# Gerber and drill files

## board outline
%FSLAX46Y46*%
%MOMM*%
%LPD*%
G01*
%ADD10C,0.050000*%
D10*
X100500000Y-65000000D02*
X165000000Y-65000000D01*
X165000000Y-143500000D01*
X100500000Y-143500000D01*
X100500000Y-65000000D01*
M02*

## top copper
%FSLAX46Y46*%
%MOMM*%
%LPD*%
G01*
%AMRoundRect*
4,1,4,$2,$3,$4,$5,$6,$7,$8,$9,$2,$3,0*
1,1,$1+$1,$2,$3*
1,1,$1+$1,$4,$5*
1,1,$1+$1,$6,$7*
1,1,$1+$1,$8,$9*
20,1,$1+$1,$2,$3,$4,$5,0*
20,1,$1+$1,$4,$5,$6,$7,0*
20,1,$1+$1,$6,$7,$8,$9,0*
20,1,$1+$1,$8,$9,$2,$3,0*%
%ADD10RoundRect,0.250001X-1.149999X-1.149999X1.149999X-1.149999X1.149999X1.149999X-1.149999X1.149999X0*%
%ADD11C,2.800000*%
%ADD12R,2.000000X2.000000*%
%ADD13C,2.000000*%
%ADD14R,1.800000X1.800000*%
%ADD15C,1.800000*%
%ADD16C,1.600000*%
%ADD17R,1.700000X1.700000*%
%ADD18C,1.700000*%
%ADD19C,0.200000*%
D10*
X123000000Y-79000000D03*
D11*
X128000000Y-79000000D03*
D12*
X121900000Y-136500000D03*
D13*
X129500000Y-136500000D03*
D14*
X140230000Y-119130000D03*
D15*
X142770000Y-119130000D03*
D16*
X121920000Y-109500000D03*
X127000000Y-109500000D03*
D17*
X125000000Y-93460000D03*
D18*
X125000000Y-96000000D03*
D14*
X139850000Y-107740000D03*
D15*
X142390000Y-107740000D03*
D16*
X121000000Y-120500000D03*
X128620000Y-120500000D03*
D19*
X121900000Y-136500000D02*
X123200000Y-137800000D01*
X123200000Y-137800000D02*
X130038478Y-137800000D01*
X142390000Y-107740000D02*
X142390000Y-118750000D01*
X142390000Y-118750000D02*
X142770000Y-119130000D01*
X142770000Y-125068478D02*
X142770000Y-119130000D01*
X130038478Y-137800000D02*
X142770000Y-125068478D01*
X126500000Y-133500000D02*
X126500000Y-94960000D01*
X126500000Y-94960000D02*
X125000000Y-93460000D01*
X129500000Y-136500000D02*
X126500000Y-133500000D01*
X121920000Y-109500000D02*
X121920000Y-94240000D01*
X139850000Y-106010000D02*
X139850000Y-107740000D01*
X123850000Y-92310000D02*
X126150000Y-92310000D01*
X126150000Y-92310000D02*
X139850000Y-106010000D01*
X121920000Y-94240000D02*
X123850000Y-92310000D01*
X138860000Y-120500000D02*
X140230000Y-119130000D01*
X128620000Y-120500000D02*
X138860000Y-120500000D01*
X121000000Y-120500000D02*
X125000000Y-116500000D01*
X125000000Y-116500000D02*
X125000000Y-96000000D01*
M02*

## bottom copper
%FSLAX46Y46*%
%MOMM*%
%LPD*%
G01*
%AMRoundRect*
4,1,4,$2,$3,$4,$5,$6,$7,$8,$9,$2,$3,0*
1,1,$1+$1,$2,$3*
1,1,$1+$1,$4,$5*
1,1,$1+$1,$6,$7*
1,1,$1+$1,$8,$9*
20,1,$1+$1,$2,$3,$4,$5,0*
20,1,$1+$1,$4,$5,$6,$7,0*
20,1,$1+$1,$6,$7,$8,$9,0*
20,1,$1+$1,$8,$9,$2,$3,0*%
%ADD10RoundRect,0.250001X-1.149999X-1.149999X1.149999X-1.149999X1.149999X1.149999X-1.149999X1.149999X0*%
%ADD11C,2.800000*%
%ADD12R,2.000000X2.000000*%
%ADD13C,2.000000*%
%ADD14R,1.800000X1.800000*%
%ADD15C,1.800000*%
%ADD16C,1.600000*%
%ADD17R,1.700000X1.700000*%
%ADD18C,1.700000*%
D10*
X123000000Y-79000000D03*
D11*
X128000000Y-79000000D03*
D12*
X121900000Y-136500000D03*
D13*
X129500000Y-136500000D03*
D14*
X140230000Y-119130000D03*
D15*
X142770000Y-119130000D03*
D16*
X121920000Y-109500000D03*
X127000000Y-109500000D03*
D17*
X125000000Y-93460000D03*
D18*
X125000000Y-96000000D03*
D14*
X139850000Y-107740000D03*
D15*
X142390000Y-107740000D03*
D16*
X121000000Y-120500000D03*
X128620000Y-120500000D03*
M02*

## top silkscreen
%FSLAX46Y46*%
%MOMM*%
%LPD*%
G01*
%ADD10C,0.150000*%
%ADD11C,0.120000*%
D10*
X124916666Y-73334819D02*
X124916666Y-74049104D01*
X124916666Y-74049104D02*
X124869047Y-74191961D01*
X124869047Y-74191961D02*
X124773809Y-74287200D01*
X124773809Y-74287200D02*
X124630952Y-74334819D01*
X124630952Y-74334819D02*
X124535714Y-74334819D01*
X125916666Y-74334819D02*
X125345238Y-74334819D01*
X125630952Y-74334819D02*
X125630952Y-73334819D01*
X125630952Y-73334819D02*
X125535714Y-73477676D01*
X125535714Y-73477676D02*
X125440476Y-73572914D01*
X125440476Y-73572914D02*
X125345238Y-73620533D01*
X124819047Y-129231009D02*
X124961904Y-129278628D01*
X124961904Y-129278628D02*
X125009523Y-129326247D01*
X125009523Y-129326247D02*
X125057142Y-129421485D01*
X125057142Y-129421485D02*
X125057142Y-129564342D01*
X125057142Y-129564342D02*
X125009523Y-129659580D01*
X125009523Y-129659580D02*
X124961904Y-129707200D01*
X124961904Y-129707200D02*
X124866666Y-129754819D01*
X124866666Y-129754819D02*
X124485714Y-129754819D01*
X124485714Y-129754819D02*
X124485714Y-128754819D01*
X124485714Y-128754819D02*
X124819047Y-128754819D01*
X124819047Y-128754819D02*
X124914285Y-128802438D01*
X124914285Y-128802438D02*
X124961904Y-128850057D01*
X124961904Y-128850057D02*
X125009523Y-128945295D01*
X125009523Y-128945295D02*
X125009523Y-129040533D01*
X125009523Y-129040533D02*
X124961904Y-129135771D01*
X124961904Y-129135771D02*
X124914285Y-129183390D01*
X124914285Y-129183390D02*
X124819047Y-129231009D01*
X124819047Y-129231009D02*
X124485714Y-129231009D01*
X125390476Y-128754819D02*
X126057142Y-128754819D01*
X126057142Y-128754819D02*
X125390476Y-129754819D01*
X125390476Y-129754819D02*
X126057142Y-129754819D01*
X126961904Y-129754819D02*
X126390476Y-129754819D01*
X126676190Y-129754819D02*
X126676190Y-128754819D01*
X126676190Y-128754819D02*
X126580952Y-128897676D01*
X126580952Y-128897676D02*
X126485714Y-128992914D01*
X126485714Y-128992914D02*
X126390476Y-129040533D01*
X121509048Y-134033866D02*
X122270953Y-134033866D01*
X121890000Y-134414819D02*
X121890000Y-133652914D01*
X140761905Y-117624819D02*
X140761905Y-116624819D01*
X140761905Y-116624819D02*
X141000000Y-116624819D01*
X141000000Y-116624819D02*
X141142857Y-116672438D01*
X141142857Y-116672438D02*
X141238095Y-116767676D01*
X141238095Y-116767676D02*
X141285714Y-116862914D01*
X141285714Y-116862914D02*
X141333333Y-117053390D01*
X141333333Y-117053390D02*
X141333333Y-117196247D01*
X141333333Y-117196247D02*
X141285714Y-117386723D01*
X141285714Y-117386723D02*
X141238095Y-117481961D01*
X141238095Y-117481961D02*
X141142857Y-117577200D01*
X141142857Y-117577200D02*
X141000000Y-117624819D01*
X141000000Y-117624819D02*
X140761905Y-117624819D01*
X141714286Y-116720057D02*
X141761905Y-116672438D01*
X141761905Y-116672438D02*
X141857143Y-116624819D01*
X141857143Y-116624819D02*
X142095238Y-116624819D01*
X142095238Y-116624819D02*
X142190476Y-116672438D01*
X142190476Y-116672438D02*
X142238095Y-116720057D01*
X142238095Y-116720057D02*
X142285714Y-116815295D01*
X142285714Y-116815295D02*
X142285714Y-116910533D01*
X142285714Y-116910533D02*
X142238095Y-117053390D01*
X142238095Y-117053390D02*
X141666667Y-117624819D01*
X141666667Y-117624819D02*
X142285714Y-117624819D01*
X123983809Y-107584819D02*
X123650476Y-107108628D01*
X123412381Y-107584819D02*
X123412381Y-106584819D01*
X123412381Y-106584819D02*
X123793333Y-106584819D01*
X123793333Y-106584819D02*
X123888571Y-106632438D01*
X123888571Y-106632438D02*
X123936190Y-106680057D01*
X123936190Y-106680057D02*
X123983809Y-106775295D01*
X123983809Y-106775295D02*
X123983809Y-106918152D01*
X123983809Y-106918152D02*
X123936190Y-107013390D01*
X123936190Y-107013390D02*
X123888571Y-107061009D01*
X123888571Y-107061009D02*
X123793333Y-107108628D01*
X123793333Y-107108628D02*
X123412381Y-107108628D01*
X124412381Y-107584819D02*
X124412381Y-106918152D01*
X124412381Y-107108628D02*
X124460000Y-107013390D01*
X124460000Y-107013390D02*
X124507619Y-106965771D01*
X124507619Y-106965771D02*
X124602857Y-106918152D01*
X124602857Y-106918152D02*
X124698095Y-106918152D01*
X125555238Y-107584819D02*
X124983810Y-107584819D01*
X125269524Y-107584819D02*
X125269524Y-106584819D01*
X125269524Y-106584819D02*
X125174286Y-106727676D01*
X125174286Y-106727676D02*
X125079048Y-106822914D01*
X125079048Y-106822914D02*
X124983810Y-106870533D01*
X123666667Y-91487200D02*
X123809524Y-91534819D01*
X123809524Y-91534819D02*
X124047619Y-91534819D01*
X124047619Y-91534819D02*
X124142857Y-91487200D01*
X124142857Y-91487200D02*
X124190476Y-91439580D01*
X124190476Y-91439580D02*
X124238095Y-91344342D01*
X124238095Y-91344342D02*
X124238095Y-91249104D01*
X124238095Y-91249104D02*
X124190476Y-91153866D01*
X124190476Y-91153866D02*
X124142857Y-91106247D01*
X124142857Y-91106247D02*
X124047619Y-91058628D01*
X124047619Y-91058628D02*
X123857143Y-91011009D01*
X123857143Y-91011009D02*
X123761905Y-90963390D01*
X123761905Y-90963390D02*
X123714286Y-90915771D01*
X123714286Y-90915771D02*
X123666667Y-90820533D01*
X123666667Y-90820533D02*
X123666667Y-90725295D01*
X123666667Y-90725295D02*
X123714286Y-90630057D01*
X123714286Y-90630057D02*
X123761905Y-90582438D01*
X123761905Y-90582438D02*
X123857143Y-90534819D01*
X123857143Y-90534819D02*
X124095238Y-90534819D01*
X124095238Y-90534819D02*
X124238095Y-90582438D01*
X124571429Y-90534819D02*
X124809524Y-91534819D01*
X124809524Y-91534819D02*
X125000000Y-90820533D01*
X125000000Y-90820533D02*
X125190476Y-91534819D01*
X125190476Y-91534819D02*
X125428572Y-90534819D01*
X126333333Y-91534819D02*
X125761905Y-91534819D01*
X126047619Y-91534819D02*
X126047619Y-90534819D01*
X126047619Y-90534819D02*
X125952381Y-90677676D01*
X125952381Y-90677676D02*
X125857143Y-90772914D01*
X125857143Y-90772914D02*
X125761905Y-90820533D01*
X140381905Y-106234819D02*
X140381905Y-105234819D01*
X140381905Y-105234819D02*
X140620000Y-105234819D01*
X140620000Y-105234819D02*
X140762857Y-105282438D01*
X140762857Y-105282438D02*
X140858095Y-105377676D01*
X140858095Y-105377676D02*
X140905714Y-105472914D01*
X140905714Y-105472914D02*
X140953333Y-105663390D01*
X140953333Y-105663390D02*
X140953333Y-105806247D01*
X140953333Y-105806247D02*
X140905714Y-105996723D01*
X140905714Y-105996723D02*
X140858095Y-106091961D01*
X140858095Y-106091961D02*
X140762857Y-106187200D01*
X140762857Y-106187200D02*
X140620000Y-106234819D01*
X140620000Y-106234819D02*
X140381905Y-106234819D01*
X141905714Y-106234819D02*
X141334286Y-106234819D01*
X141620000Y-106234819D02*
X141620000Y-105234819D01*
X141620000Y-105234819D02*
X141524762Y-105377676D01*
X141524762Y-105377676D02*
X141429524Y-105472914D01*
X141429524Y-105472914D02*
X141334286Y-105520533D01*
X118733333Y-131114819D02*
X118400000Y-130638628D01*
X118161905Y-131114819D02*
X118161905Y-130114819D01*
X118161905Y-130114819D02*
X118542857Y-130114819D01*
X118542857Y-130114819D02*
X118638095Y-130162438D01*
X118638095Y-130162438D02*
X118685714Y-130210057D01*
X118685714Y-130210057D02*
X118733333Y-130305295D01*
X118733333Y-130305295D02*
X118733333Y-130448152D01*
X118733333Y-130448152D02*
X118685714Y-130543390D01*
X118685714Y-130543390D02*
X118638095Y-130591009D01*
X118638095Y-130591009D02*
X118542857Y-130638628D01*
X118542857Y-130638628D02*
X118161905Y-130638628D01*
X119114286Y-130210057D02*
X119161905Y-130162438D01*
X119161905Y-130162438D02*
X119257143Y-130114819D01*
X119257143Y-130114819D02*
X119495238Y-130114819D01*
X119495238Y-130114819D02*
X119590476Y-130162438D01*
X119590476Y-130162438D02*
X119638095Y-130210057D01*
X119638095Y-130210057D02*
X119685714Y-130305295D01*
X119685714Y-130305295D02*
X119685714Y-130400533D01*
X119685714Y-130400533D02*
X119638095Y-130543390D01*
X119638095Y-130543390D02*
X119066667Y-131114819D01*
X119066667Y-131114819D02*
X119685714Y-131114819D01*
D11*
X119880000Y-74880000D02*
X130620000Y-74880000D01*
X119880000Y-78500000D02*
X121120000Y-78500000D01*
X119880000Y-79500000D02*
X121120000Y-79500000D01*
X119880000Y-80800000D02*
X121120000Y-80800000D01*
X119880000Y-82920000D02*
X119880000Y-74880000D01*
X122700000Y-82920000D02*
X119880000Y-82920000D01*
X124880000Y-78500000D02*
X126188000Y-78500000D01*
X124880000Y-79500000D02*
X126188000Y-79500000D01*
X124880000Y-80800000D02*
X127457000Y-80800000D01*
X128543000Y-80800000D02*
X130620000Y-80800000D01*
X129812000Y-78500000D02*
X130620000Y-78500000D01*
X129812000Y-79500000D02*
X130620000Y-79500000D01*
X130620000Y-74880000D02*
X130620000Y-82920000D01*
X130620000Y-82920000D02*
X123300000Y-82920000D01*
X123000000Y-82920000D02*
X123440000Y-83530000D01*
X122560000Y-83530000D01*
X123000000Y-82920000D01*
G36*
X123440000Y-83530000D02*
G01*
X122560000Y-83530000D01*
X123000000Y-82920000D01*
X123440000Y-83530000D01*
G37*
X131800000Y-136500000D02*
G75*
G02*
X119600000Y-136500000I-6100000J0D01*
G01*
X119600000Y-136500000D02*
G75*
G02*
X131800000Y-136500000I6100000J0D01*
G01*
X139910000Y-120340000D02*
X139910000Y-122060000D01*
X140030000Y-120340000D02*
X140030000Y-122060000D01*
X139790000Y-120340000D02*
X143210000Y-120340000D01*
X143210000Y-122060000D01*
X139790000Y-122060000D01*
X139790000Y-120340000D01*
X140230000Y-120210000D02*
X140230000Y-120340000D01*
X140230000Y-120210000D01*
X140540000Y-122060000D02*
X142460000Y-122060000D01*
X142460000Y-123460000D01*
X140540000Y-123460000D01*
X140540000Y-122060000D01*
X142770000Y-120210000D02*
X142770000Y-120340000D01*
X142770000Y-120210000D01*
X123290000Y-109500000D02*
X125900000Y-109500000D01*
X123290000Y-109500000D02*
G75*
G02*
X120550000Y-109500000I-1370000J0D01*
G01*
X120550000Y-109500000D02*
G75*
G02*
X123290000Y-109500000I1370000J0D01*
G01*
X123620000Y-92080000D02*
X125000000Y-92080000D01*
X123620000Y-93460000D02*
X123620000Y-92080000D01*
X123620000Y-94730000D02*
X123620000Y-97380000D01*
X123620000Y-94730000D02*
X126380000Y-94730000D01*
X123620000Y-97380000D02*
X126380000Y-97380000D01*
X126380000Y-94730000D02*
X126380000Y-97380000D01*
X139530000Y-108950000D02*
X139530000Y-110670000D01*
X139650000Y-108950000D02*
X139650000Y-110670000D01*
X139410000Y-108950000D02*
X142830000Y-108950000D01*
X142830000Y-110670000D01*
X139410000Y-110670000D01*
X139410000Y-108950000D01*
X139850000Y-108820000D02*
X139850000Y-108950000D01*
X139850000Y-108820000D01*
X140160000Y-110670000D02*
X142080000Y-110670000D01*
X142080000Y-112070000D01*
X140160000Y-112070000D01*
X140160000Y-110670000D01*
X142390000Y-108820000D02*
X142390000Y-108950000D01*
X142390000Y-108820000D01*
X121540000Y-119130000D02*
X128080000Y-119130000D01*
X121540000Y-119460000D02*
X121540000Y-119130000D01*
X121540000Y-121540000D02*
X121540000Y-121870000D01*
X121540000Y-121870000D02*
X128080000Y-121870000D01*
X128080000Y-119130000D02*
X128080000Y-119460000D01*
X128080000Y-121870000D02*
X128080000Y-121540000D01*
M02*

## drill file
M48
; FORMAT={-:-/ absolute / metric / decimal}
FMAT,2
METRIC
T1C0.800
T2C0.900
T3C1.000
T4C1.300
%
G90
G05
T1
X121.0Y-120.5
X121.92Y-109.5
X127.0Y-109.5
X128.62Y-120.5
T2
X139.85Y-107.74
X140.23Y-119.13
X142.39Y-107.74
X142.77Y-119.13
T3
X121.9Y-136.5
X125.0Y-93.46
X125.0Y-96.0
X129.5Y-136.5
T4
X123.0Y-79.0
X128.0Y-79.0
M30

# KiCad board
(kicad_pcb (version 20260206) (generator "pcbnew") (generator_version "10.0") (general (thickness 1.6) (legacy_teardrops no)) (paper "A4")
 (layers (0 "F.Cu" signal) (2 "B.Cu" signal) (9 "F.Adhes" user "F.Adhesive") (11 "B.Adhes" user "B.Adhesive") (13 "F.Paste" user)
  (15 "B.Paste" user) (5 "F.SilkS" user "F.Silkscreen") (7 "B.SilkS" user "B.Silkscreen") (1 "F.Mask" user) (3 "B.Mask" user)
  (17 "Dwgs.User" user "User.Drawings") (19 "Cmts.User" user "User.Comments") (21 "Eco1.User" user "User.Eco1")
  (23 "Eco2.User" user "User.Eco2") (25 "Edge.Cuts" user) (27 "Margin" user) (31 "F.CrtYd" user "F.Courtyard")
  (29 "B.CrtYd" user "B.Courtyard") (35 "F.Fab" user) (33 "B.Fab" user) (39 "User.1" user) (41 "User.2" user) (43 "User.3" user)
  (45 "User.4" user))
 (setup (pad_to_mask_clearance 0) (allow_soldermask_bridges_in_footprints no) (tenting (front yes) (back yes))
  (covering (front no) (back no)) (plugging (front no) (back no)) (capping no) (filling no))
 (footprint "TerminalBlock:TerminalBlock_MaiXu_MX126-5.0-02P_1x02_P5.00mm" (layer "F.Cu") (at 123 79)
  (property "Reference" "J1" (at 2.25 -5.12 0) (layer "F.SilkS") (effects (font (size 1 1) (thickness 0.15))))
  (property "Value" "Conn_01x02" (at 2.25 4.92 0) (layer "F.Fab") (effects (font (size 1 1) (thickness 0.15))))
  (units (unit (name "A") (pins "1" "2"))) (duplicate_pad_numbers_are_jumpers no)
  (fp_line (start -3.12 -4.12) (end 7.62 -4.12) (stroke (width 0.12) (type solid)) (layer "F.SilkS"))
  (fp_line (start -3.12 -0.5) (end -1.88 -0.5) (stroke (width 0.12) (type solid)) (layer "F.SilkS"))
  (fp_line (start -3.12 0.5) (end -1.88 0.5) (stroke (width 0.12) (type solid)) (layer "F.SilkS"))
  (fp_line (start -3.12 1.8) (end -1.88 1.8) (stroke (width 0.12) (type solid)) (layer "F.SilkS"))
  (fp_line (start -3.12 3.92) (end -3.12 -4.12) (stroke (width 0.12) (type solid)) (layer "F.SilkS"))
  (fp_line (start -0.3 3.92) (end -3.12 3.92) (stroke (width 0.12) (type solid)) (layer "F.SilkS"))
  (fp_line (start 1.88 -0.5) (end 3.188 -0.5) (stroke (width 0.12) (type solid)) (layer "F.SilkS"))
  (fp_line (start 1.88 0.5) (end 3.188 0.5) (stroke (width 0.12) (type solid)) (layer "F.SilkS"))
  (fp_line (start 1.88 1.8) (end 4.457 1.8) (stroke (width 0.12) (type solid)) (layer "F.SilkS"))
  (fp_line (start 5.543 1.8) (end 7.62 1.8) (stroke (width 0.12) (type solid)) (layer "F.SilkS"))
  (fp_line (start 6.812 -0.5) (end 7.62 -0.5) (stroke (width 0.12) (type solid)) (layer "F.SilkS"))
  (fp_line (start 6.812 0.5) (end 7.62 0.5) (stroke (width 0.12) (type solid)) (layer "F.SilkS"))
  (fp_line (start 7.62 -4.12) (end 7.62 3.92) (stroke (width 0.12) (type solid)) (layer "F.SilkS"))
  (fp_line (start 7.62 3.92) (end 0.3 3.92) (stroke (width 0.12) (type solid)) (layer "F.SilkS"))
  (fp_poly (pts (xy 0 3.92) (xy 0.44 4.53) (xy -0.44 4.53)) (stroke (width 0.12) (type solid)) (fill yes) (layer "F.SilkS"))
  (pad "1" thru_hole roundrect (at 0 0) (size 2.8 2.8) (drill 1.3) (layers "*.Cu" "*.Mask") (remove_unused_layers no)
   (roundrect_rratio 0.089286) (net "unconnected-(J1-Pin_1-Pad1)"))
  (pad "2" thru_hole circle (at 5 0) (size 2.8 2.8) (drill 1.3) (layers "*.Cu" "*.Mask") (remove_unused_layers no)
   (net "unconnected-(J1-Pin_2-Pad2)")))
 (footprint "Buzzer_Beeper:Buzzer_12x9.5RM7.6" (layer "F.Cu") (at 121.9 136.5)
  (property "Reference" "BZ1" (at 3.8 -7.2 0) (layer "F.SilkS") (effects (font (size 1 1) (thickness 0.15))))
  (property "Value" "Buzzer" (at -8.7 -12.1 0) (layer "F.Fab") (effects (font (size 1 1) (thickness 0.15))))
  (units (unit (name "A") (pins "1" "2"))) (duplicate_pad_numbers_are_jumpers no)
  (fp_circle (center 3.8 0) (end 9.9 0) (stroke (width 0.12) (type solid)) (fill no) (layer "F.SilkS"))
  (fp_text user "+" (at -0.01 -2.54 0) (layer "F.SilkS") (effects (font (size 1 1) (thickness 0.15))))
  (pad "1" thru_hole rect (at 0 0) (size 2 2) (drill 1) (layers "*.Cu" "*.Mask") (remove_unused_layers no) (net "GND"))
  (pad "2" thru_hole circle (at 7.6 0) (size 2 2) (drill 1) (layers "*.Cu" "*.Mask") (remove_unused_layers no) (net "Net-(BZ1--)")))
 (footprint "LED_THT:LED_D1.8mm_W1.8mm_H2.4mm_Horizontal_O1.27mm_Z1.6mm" (layer "F.Cu") (at 140.23 119.13)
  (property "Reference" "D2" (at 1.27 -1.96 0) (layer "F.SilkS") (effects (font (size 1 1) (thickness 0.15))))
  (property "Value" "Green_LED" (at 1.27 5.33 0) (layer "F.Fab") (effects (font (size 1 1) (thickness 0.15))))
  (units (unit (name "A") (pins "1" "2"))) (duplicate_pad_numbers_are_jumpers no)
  (fp_line (start -0.32 1.21) (end -0.32 2.93) (stroke (width 0.12) (type solid)) (layer "F.SilkS"))
  (fp_line (start -0.2 1.21) (end -0.2 2.93) (stroke (width 0.12) (type solid)) (layer "F.SilkS"))
  (fp_rect (start -0.44 1.21) (end 2.98 2.93) (stroke (width 0.12) (type solid)) (fill no) (layer "F.SilkS"))
  (fp_rect (start 0 1.08) (end 0 1.21) (stroke (width 0.12) (type solid)) (fill no) (layer "F.SilkS"))
  (fp_rect (start 0.31 2.93) (end 2.23 4.33) (stroke (width 0.12) (type solid)) (fill no) (layer "F.SilkS"))
  (fp_rect (start 2.54 1.08) (end 2.54 1.21) (stroke (width 0.12) (type solid)) (fill no) (layer "F.SilkS"))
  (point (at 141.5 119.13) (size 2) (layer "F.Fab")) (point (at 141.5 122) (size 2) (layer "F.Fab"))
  (pad "1" thru_hole rect (at 0 0) (size 1.8 1.8) (drill 0.9) (layers "*.Cu" "*.Mask") (remove_unused_layers no) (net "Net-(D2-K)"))
  (pad "2" thru_hole circle (at 2.54 0) (size 1.8 1.8) (drill 0.9) (layers "*.Cu" "*.Mask") (remove_unused_layers no) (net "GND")))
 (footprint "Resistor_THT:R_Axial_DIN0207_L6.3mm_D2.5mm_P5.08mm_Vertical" (layer "F.Cu") (at 121.92 109.5)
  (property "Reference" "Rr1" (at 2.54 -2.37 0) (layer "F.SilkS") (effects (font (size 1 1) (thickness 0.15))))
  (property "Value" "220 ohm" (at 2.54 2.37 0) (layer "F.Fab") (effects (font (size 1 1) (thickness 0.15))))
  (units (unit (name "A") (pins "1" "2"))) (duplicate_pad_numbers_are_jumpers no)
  (fp_line (start 1.37 0) (end 3.98 0) (stroke (width 0.12) (type solid)) (layer "F.SilkS"))
  (fp_circle (center 0 0) (end 1.37 0) (stroke (width 0.12) (type solid)) (fill no) (layer "F.SilkS"))
  (pad "1" thru_hole circle (at 0 0) (size 1.6 1.6) (drill 0.8) (layers "*.Cu" "*.Mask") (remove_unused_layers no) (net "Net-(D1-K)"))
  (pad "2" thru_hole circle (at 5.08 0) (size 1.6 1.6) (drill 0.8) (layers "*.Cu" "*.Mask") (remove_unused_layers no) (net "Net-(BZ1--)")))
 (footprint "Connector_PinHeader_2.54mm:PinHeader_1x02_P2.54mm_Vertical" (layer "F.Cu") (at 125 93.46)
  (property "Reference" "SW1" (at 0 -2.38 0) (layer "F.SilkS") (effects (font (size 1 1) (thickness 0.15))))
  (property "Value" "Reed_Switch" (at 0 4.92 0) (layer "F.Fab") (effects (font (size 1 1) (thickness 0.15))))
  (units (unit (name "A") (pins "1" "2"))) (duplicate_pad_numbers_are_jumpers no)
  (fp_line (start -1.38 -1.38) (end 0 -1.38) (stroke (width 0.12) (type solid)) (layer "F.SilkS"))
  (fp_line (start -1.38 0) (end -1.38 -1.38) (stroke (width 0.12) (type solid)) (layer "F.SilkS"))
  (fp_line (start -1.38 1.27) (end -1.38 3.92) (stroke (width 0.12) (type solid)) (layer "F.SilkS"))
  (fp_line (start -1.38 1.27) (end 1.38 1.27) (stroke (width 0.12) (type solid)) (layer "F.SilkS"))
  (fp_line (start -1.38 3.92) (end 1.38 3.92) (stroke (width 0.12) (type solid)) (layer "F.SilkS"))
  (fp_line (start 1.38 1.27) (end 1.38 3.92) (stroke (width 0.12) (type solid)) (layer "F.SilkS"))
  (pad "1" thru_hole rect (at 0 0) (size 1.7 1.7) (drill 1) (layers "*.Cu" "*.Mask") (remove_unused_layers no) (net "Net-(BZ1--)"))
  (pad "2" thru_hole circle (at 0 2.54) (size 1.7 1.7) (drill 1) (layers "*.Cu" "*.Mask") (remove_unused_layers no) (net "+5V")))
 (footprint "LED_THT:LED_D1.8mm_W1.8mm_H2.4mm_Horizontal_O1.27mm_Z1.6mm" (layer "F.Cu") (at 139.85 107.74)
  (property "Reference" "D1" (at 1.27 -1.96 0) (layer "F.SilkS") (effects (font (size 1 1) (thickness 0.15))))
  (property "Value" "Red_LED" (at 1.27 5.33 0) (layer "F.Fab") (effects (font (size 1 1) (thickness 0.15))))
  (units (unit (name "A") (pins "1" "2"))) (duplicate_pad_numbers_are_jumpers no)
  (fp_line (start -0.32 1.21) (end -0.32 2.93) (stroke (width 0.12) (type solid)) (layer "F.SilkS"))
  (fp_line (start -0.2 1.21) (end -0.2 2.93) (stroke (width 0.12) (type solid)) (layer "F.SilkS"))
  (fp_rect (start -0.44 1.21) (end 2.98 2.93) (stroke (width 0.12) (type solid)) (fill no) (layer "F.SilkS"))
  (fp_rect (start 0 1.08) (end 0 1.21) (stroke (width 0.12) (type solid)) (fill no) (layer "F.SilkS"))
  (fp_rect (start 0.31 2.93) (end 2.23 4.33) (stroke (width 0.12) (type solid)) (fill no) (layer "F.SilkS"))
  (fp_rect (start 2.54 1.08) (end 2.54 1.21) (stroke (width 0.12) (type solid)) (fill no) (layer "F.SilkS"))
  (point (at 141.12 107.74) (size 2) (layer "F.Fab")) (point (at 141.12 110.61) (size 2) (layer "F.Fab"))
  (pad "1" thru_hole rect (at 0 0) (size 1.8 1.8) (drill 0.9) (layers "*.Cu" "*.Mask") (remove_unused_layers no) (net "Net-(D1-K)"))
  (pad "2" thru_hole circle (at 2.54 0) (size 1.8 1.8) (drill 0.9) (layers "*.Cu" "*.Mask") (remove_unused_layers no) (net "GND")))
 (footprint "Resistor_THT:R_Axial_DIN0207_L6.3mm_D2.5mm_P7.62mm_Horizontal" (layer "F.Cu") (at 121 120.5)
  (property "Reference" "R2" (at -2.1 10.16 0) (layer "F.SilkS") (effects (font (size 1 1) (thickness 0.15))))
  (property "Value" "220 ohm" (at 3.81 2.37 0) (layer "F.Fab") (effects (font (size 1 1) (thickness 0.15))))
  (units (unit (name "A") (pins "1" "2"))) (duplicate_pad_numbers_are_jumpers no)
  (fp_line (start 0.54 -1.37) (end 7.08 -1.37) (stroke (width 0.12) (type solid)) (layer "F.SilkS"))
  (fp_line (start 0.54 -1.04) (end 0.54 -1.37) (stroke (width 0.12) (type solid)) (layer "F.SilkS"))
  (fp_line (start 0.54 1.04) (end 0.54 1.37) (stroke (width 0.12) (type solid)) (layer "F.SilkS"))
  (fp_line (start 0.54 1.37) (end 7.08 1.37) (stroke (width 0.12) (type solid)) (layer "F.SilkS"))
  (fp_line (start 7.08 -1.37) (end 7.08 -1.04) (stroke (width 0.12) (type solid)) (layer "F.SilkS"))
  (fp_line (start 7.08 1.37) (end 7.08 1.04) (stroke (width 0.12) (type solid)) (layer "F.SilkS"))
  (pad "1" thru_hole circle (at 0 0) (size 1.6 1.6) (drill 0.8) (layers "*.Cu" "*.Mask") (remove_unused_layers no) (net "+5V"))
  (pad "2" thru_hole circle (at 7.62 0) (size 1.6 1.6) (drill 0.8) (layers "*.Cu" "*.Mask") (remove_unused_layers no) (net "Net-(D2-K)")))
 (gr_rect (start 100.5 65) (end 165 143.5) (stroke (width 0.05) (type default)) (fill no) (layer "Edge.Cuts"))
 (segment (start 121.9 136.5) (end 123.2 137.8) (width 0.2) (layer "F.Cu") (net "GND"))
 (segment (start 123.2 137.8) (end 130.038478 137.8) (width 0.2) (layer "F.Cu") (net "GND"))
 (segment (start 142.39 107.74) (end 142.39 118.75) (width 0.2) (layer "F.Cu") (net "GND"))
 (segment (start 142.39 118.75) (end 142.77 119.13) (width 0.2) (layer "F.Cu") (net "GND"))
 (segment (start 142.77 125.068478) (end 142.77 119.13) (width 0.2) (layer "F.Cu") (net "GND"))
 (segment (start 130.038478 137.8) (end 142.77 125.068478) (width 0.2) (layer "F.Cu") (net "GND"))
 (segment (start 126.5 133.5) (end 126.5 94.96) (width 0.2) (layer "F.Cu") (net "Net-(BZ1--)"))
 (segment (start 126.5 94.96) (end 125 93.46) (width 0.2) (layer "F.Cu") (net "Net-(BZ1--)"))
 (segment (start 129.5 136.5) (end 126.5 133.5) (width 0.2) (layer "F.Cu") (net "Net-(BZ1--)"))
 (segment (start 121.92 109.5) (end 121.92 94.24) (width 0.2) (layer "F.Cu") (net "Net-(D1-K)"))
 (segment (start 139.85 106.01) (end 139.85 107.74) (width 0.2) (layer "F.Cu") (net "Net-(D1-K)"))
 (segment (start 123.85 92.31) (end 126.15 92.31) (width 0.2) (layer "F.Cu") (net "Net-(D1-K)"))
 (segment (start 126.15 92.31) (end 139.85 106.01) (width 0.2) (layer "F.Cu") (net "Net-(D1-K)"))
 (segment (start 121.92 94.24) (end 123.85 92.31) (width 0.2) (layer "F.Cu") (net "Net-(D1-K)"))
 (segment (start 138.86 120.5) (end 140.23 119.13) (width 0.2) (layer "F.Cu") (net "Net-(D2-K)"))
 (segment (start 128.62 120.5) (end 138.86 120.5) (width 0.2) (layer "F.Cu") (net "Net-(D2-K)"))
 (segment (start 121 120.5) (end 125 116.5) (width 0.2) (layer "F.Cu") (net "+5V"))
 (segment (start 125 116.5) (end 125 96) (width 0.2) (layer "F.Cu") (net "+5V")))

